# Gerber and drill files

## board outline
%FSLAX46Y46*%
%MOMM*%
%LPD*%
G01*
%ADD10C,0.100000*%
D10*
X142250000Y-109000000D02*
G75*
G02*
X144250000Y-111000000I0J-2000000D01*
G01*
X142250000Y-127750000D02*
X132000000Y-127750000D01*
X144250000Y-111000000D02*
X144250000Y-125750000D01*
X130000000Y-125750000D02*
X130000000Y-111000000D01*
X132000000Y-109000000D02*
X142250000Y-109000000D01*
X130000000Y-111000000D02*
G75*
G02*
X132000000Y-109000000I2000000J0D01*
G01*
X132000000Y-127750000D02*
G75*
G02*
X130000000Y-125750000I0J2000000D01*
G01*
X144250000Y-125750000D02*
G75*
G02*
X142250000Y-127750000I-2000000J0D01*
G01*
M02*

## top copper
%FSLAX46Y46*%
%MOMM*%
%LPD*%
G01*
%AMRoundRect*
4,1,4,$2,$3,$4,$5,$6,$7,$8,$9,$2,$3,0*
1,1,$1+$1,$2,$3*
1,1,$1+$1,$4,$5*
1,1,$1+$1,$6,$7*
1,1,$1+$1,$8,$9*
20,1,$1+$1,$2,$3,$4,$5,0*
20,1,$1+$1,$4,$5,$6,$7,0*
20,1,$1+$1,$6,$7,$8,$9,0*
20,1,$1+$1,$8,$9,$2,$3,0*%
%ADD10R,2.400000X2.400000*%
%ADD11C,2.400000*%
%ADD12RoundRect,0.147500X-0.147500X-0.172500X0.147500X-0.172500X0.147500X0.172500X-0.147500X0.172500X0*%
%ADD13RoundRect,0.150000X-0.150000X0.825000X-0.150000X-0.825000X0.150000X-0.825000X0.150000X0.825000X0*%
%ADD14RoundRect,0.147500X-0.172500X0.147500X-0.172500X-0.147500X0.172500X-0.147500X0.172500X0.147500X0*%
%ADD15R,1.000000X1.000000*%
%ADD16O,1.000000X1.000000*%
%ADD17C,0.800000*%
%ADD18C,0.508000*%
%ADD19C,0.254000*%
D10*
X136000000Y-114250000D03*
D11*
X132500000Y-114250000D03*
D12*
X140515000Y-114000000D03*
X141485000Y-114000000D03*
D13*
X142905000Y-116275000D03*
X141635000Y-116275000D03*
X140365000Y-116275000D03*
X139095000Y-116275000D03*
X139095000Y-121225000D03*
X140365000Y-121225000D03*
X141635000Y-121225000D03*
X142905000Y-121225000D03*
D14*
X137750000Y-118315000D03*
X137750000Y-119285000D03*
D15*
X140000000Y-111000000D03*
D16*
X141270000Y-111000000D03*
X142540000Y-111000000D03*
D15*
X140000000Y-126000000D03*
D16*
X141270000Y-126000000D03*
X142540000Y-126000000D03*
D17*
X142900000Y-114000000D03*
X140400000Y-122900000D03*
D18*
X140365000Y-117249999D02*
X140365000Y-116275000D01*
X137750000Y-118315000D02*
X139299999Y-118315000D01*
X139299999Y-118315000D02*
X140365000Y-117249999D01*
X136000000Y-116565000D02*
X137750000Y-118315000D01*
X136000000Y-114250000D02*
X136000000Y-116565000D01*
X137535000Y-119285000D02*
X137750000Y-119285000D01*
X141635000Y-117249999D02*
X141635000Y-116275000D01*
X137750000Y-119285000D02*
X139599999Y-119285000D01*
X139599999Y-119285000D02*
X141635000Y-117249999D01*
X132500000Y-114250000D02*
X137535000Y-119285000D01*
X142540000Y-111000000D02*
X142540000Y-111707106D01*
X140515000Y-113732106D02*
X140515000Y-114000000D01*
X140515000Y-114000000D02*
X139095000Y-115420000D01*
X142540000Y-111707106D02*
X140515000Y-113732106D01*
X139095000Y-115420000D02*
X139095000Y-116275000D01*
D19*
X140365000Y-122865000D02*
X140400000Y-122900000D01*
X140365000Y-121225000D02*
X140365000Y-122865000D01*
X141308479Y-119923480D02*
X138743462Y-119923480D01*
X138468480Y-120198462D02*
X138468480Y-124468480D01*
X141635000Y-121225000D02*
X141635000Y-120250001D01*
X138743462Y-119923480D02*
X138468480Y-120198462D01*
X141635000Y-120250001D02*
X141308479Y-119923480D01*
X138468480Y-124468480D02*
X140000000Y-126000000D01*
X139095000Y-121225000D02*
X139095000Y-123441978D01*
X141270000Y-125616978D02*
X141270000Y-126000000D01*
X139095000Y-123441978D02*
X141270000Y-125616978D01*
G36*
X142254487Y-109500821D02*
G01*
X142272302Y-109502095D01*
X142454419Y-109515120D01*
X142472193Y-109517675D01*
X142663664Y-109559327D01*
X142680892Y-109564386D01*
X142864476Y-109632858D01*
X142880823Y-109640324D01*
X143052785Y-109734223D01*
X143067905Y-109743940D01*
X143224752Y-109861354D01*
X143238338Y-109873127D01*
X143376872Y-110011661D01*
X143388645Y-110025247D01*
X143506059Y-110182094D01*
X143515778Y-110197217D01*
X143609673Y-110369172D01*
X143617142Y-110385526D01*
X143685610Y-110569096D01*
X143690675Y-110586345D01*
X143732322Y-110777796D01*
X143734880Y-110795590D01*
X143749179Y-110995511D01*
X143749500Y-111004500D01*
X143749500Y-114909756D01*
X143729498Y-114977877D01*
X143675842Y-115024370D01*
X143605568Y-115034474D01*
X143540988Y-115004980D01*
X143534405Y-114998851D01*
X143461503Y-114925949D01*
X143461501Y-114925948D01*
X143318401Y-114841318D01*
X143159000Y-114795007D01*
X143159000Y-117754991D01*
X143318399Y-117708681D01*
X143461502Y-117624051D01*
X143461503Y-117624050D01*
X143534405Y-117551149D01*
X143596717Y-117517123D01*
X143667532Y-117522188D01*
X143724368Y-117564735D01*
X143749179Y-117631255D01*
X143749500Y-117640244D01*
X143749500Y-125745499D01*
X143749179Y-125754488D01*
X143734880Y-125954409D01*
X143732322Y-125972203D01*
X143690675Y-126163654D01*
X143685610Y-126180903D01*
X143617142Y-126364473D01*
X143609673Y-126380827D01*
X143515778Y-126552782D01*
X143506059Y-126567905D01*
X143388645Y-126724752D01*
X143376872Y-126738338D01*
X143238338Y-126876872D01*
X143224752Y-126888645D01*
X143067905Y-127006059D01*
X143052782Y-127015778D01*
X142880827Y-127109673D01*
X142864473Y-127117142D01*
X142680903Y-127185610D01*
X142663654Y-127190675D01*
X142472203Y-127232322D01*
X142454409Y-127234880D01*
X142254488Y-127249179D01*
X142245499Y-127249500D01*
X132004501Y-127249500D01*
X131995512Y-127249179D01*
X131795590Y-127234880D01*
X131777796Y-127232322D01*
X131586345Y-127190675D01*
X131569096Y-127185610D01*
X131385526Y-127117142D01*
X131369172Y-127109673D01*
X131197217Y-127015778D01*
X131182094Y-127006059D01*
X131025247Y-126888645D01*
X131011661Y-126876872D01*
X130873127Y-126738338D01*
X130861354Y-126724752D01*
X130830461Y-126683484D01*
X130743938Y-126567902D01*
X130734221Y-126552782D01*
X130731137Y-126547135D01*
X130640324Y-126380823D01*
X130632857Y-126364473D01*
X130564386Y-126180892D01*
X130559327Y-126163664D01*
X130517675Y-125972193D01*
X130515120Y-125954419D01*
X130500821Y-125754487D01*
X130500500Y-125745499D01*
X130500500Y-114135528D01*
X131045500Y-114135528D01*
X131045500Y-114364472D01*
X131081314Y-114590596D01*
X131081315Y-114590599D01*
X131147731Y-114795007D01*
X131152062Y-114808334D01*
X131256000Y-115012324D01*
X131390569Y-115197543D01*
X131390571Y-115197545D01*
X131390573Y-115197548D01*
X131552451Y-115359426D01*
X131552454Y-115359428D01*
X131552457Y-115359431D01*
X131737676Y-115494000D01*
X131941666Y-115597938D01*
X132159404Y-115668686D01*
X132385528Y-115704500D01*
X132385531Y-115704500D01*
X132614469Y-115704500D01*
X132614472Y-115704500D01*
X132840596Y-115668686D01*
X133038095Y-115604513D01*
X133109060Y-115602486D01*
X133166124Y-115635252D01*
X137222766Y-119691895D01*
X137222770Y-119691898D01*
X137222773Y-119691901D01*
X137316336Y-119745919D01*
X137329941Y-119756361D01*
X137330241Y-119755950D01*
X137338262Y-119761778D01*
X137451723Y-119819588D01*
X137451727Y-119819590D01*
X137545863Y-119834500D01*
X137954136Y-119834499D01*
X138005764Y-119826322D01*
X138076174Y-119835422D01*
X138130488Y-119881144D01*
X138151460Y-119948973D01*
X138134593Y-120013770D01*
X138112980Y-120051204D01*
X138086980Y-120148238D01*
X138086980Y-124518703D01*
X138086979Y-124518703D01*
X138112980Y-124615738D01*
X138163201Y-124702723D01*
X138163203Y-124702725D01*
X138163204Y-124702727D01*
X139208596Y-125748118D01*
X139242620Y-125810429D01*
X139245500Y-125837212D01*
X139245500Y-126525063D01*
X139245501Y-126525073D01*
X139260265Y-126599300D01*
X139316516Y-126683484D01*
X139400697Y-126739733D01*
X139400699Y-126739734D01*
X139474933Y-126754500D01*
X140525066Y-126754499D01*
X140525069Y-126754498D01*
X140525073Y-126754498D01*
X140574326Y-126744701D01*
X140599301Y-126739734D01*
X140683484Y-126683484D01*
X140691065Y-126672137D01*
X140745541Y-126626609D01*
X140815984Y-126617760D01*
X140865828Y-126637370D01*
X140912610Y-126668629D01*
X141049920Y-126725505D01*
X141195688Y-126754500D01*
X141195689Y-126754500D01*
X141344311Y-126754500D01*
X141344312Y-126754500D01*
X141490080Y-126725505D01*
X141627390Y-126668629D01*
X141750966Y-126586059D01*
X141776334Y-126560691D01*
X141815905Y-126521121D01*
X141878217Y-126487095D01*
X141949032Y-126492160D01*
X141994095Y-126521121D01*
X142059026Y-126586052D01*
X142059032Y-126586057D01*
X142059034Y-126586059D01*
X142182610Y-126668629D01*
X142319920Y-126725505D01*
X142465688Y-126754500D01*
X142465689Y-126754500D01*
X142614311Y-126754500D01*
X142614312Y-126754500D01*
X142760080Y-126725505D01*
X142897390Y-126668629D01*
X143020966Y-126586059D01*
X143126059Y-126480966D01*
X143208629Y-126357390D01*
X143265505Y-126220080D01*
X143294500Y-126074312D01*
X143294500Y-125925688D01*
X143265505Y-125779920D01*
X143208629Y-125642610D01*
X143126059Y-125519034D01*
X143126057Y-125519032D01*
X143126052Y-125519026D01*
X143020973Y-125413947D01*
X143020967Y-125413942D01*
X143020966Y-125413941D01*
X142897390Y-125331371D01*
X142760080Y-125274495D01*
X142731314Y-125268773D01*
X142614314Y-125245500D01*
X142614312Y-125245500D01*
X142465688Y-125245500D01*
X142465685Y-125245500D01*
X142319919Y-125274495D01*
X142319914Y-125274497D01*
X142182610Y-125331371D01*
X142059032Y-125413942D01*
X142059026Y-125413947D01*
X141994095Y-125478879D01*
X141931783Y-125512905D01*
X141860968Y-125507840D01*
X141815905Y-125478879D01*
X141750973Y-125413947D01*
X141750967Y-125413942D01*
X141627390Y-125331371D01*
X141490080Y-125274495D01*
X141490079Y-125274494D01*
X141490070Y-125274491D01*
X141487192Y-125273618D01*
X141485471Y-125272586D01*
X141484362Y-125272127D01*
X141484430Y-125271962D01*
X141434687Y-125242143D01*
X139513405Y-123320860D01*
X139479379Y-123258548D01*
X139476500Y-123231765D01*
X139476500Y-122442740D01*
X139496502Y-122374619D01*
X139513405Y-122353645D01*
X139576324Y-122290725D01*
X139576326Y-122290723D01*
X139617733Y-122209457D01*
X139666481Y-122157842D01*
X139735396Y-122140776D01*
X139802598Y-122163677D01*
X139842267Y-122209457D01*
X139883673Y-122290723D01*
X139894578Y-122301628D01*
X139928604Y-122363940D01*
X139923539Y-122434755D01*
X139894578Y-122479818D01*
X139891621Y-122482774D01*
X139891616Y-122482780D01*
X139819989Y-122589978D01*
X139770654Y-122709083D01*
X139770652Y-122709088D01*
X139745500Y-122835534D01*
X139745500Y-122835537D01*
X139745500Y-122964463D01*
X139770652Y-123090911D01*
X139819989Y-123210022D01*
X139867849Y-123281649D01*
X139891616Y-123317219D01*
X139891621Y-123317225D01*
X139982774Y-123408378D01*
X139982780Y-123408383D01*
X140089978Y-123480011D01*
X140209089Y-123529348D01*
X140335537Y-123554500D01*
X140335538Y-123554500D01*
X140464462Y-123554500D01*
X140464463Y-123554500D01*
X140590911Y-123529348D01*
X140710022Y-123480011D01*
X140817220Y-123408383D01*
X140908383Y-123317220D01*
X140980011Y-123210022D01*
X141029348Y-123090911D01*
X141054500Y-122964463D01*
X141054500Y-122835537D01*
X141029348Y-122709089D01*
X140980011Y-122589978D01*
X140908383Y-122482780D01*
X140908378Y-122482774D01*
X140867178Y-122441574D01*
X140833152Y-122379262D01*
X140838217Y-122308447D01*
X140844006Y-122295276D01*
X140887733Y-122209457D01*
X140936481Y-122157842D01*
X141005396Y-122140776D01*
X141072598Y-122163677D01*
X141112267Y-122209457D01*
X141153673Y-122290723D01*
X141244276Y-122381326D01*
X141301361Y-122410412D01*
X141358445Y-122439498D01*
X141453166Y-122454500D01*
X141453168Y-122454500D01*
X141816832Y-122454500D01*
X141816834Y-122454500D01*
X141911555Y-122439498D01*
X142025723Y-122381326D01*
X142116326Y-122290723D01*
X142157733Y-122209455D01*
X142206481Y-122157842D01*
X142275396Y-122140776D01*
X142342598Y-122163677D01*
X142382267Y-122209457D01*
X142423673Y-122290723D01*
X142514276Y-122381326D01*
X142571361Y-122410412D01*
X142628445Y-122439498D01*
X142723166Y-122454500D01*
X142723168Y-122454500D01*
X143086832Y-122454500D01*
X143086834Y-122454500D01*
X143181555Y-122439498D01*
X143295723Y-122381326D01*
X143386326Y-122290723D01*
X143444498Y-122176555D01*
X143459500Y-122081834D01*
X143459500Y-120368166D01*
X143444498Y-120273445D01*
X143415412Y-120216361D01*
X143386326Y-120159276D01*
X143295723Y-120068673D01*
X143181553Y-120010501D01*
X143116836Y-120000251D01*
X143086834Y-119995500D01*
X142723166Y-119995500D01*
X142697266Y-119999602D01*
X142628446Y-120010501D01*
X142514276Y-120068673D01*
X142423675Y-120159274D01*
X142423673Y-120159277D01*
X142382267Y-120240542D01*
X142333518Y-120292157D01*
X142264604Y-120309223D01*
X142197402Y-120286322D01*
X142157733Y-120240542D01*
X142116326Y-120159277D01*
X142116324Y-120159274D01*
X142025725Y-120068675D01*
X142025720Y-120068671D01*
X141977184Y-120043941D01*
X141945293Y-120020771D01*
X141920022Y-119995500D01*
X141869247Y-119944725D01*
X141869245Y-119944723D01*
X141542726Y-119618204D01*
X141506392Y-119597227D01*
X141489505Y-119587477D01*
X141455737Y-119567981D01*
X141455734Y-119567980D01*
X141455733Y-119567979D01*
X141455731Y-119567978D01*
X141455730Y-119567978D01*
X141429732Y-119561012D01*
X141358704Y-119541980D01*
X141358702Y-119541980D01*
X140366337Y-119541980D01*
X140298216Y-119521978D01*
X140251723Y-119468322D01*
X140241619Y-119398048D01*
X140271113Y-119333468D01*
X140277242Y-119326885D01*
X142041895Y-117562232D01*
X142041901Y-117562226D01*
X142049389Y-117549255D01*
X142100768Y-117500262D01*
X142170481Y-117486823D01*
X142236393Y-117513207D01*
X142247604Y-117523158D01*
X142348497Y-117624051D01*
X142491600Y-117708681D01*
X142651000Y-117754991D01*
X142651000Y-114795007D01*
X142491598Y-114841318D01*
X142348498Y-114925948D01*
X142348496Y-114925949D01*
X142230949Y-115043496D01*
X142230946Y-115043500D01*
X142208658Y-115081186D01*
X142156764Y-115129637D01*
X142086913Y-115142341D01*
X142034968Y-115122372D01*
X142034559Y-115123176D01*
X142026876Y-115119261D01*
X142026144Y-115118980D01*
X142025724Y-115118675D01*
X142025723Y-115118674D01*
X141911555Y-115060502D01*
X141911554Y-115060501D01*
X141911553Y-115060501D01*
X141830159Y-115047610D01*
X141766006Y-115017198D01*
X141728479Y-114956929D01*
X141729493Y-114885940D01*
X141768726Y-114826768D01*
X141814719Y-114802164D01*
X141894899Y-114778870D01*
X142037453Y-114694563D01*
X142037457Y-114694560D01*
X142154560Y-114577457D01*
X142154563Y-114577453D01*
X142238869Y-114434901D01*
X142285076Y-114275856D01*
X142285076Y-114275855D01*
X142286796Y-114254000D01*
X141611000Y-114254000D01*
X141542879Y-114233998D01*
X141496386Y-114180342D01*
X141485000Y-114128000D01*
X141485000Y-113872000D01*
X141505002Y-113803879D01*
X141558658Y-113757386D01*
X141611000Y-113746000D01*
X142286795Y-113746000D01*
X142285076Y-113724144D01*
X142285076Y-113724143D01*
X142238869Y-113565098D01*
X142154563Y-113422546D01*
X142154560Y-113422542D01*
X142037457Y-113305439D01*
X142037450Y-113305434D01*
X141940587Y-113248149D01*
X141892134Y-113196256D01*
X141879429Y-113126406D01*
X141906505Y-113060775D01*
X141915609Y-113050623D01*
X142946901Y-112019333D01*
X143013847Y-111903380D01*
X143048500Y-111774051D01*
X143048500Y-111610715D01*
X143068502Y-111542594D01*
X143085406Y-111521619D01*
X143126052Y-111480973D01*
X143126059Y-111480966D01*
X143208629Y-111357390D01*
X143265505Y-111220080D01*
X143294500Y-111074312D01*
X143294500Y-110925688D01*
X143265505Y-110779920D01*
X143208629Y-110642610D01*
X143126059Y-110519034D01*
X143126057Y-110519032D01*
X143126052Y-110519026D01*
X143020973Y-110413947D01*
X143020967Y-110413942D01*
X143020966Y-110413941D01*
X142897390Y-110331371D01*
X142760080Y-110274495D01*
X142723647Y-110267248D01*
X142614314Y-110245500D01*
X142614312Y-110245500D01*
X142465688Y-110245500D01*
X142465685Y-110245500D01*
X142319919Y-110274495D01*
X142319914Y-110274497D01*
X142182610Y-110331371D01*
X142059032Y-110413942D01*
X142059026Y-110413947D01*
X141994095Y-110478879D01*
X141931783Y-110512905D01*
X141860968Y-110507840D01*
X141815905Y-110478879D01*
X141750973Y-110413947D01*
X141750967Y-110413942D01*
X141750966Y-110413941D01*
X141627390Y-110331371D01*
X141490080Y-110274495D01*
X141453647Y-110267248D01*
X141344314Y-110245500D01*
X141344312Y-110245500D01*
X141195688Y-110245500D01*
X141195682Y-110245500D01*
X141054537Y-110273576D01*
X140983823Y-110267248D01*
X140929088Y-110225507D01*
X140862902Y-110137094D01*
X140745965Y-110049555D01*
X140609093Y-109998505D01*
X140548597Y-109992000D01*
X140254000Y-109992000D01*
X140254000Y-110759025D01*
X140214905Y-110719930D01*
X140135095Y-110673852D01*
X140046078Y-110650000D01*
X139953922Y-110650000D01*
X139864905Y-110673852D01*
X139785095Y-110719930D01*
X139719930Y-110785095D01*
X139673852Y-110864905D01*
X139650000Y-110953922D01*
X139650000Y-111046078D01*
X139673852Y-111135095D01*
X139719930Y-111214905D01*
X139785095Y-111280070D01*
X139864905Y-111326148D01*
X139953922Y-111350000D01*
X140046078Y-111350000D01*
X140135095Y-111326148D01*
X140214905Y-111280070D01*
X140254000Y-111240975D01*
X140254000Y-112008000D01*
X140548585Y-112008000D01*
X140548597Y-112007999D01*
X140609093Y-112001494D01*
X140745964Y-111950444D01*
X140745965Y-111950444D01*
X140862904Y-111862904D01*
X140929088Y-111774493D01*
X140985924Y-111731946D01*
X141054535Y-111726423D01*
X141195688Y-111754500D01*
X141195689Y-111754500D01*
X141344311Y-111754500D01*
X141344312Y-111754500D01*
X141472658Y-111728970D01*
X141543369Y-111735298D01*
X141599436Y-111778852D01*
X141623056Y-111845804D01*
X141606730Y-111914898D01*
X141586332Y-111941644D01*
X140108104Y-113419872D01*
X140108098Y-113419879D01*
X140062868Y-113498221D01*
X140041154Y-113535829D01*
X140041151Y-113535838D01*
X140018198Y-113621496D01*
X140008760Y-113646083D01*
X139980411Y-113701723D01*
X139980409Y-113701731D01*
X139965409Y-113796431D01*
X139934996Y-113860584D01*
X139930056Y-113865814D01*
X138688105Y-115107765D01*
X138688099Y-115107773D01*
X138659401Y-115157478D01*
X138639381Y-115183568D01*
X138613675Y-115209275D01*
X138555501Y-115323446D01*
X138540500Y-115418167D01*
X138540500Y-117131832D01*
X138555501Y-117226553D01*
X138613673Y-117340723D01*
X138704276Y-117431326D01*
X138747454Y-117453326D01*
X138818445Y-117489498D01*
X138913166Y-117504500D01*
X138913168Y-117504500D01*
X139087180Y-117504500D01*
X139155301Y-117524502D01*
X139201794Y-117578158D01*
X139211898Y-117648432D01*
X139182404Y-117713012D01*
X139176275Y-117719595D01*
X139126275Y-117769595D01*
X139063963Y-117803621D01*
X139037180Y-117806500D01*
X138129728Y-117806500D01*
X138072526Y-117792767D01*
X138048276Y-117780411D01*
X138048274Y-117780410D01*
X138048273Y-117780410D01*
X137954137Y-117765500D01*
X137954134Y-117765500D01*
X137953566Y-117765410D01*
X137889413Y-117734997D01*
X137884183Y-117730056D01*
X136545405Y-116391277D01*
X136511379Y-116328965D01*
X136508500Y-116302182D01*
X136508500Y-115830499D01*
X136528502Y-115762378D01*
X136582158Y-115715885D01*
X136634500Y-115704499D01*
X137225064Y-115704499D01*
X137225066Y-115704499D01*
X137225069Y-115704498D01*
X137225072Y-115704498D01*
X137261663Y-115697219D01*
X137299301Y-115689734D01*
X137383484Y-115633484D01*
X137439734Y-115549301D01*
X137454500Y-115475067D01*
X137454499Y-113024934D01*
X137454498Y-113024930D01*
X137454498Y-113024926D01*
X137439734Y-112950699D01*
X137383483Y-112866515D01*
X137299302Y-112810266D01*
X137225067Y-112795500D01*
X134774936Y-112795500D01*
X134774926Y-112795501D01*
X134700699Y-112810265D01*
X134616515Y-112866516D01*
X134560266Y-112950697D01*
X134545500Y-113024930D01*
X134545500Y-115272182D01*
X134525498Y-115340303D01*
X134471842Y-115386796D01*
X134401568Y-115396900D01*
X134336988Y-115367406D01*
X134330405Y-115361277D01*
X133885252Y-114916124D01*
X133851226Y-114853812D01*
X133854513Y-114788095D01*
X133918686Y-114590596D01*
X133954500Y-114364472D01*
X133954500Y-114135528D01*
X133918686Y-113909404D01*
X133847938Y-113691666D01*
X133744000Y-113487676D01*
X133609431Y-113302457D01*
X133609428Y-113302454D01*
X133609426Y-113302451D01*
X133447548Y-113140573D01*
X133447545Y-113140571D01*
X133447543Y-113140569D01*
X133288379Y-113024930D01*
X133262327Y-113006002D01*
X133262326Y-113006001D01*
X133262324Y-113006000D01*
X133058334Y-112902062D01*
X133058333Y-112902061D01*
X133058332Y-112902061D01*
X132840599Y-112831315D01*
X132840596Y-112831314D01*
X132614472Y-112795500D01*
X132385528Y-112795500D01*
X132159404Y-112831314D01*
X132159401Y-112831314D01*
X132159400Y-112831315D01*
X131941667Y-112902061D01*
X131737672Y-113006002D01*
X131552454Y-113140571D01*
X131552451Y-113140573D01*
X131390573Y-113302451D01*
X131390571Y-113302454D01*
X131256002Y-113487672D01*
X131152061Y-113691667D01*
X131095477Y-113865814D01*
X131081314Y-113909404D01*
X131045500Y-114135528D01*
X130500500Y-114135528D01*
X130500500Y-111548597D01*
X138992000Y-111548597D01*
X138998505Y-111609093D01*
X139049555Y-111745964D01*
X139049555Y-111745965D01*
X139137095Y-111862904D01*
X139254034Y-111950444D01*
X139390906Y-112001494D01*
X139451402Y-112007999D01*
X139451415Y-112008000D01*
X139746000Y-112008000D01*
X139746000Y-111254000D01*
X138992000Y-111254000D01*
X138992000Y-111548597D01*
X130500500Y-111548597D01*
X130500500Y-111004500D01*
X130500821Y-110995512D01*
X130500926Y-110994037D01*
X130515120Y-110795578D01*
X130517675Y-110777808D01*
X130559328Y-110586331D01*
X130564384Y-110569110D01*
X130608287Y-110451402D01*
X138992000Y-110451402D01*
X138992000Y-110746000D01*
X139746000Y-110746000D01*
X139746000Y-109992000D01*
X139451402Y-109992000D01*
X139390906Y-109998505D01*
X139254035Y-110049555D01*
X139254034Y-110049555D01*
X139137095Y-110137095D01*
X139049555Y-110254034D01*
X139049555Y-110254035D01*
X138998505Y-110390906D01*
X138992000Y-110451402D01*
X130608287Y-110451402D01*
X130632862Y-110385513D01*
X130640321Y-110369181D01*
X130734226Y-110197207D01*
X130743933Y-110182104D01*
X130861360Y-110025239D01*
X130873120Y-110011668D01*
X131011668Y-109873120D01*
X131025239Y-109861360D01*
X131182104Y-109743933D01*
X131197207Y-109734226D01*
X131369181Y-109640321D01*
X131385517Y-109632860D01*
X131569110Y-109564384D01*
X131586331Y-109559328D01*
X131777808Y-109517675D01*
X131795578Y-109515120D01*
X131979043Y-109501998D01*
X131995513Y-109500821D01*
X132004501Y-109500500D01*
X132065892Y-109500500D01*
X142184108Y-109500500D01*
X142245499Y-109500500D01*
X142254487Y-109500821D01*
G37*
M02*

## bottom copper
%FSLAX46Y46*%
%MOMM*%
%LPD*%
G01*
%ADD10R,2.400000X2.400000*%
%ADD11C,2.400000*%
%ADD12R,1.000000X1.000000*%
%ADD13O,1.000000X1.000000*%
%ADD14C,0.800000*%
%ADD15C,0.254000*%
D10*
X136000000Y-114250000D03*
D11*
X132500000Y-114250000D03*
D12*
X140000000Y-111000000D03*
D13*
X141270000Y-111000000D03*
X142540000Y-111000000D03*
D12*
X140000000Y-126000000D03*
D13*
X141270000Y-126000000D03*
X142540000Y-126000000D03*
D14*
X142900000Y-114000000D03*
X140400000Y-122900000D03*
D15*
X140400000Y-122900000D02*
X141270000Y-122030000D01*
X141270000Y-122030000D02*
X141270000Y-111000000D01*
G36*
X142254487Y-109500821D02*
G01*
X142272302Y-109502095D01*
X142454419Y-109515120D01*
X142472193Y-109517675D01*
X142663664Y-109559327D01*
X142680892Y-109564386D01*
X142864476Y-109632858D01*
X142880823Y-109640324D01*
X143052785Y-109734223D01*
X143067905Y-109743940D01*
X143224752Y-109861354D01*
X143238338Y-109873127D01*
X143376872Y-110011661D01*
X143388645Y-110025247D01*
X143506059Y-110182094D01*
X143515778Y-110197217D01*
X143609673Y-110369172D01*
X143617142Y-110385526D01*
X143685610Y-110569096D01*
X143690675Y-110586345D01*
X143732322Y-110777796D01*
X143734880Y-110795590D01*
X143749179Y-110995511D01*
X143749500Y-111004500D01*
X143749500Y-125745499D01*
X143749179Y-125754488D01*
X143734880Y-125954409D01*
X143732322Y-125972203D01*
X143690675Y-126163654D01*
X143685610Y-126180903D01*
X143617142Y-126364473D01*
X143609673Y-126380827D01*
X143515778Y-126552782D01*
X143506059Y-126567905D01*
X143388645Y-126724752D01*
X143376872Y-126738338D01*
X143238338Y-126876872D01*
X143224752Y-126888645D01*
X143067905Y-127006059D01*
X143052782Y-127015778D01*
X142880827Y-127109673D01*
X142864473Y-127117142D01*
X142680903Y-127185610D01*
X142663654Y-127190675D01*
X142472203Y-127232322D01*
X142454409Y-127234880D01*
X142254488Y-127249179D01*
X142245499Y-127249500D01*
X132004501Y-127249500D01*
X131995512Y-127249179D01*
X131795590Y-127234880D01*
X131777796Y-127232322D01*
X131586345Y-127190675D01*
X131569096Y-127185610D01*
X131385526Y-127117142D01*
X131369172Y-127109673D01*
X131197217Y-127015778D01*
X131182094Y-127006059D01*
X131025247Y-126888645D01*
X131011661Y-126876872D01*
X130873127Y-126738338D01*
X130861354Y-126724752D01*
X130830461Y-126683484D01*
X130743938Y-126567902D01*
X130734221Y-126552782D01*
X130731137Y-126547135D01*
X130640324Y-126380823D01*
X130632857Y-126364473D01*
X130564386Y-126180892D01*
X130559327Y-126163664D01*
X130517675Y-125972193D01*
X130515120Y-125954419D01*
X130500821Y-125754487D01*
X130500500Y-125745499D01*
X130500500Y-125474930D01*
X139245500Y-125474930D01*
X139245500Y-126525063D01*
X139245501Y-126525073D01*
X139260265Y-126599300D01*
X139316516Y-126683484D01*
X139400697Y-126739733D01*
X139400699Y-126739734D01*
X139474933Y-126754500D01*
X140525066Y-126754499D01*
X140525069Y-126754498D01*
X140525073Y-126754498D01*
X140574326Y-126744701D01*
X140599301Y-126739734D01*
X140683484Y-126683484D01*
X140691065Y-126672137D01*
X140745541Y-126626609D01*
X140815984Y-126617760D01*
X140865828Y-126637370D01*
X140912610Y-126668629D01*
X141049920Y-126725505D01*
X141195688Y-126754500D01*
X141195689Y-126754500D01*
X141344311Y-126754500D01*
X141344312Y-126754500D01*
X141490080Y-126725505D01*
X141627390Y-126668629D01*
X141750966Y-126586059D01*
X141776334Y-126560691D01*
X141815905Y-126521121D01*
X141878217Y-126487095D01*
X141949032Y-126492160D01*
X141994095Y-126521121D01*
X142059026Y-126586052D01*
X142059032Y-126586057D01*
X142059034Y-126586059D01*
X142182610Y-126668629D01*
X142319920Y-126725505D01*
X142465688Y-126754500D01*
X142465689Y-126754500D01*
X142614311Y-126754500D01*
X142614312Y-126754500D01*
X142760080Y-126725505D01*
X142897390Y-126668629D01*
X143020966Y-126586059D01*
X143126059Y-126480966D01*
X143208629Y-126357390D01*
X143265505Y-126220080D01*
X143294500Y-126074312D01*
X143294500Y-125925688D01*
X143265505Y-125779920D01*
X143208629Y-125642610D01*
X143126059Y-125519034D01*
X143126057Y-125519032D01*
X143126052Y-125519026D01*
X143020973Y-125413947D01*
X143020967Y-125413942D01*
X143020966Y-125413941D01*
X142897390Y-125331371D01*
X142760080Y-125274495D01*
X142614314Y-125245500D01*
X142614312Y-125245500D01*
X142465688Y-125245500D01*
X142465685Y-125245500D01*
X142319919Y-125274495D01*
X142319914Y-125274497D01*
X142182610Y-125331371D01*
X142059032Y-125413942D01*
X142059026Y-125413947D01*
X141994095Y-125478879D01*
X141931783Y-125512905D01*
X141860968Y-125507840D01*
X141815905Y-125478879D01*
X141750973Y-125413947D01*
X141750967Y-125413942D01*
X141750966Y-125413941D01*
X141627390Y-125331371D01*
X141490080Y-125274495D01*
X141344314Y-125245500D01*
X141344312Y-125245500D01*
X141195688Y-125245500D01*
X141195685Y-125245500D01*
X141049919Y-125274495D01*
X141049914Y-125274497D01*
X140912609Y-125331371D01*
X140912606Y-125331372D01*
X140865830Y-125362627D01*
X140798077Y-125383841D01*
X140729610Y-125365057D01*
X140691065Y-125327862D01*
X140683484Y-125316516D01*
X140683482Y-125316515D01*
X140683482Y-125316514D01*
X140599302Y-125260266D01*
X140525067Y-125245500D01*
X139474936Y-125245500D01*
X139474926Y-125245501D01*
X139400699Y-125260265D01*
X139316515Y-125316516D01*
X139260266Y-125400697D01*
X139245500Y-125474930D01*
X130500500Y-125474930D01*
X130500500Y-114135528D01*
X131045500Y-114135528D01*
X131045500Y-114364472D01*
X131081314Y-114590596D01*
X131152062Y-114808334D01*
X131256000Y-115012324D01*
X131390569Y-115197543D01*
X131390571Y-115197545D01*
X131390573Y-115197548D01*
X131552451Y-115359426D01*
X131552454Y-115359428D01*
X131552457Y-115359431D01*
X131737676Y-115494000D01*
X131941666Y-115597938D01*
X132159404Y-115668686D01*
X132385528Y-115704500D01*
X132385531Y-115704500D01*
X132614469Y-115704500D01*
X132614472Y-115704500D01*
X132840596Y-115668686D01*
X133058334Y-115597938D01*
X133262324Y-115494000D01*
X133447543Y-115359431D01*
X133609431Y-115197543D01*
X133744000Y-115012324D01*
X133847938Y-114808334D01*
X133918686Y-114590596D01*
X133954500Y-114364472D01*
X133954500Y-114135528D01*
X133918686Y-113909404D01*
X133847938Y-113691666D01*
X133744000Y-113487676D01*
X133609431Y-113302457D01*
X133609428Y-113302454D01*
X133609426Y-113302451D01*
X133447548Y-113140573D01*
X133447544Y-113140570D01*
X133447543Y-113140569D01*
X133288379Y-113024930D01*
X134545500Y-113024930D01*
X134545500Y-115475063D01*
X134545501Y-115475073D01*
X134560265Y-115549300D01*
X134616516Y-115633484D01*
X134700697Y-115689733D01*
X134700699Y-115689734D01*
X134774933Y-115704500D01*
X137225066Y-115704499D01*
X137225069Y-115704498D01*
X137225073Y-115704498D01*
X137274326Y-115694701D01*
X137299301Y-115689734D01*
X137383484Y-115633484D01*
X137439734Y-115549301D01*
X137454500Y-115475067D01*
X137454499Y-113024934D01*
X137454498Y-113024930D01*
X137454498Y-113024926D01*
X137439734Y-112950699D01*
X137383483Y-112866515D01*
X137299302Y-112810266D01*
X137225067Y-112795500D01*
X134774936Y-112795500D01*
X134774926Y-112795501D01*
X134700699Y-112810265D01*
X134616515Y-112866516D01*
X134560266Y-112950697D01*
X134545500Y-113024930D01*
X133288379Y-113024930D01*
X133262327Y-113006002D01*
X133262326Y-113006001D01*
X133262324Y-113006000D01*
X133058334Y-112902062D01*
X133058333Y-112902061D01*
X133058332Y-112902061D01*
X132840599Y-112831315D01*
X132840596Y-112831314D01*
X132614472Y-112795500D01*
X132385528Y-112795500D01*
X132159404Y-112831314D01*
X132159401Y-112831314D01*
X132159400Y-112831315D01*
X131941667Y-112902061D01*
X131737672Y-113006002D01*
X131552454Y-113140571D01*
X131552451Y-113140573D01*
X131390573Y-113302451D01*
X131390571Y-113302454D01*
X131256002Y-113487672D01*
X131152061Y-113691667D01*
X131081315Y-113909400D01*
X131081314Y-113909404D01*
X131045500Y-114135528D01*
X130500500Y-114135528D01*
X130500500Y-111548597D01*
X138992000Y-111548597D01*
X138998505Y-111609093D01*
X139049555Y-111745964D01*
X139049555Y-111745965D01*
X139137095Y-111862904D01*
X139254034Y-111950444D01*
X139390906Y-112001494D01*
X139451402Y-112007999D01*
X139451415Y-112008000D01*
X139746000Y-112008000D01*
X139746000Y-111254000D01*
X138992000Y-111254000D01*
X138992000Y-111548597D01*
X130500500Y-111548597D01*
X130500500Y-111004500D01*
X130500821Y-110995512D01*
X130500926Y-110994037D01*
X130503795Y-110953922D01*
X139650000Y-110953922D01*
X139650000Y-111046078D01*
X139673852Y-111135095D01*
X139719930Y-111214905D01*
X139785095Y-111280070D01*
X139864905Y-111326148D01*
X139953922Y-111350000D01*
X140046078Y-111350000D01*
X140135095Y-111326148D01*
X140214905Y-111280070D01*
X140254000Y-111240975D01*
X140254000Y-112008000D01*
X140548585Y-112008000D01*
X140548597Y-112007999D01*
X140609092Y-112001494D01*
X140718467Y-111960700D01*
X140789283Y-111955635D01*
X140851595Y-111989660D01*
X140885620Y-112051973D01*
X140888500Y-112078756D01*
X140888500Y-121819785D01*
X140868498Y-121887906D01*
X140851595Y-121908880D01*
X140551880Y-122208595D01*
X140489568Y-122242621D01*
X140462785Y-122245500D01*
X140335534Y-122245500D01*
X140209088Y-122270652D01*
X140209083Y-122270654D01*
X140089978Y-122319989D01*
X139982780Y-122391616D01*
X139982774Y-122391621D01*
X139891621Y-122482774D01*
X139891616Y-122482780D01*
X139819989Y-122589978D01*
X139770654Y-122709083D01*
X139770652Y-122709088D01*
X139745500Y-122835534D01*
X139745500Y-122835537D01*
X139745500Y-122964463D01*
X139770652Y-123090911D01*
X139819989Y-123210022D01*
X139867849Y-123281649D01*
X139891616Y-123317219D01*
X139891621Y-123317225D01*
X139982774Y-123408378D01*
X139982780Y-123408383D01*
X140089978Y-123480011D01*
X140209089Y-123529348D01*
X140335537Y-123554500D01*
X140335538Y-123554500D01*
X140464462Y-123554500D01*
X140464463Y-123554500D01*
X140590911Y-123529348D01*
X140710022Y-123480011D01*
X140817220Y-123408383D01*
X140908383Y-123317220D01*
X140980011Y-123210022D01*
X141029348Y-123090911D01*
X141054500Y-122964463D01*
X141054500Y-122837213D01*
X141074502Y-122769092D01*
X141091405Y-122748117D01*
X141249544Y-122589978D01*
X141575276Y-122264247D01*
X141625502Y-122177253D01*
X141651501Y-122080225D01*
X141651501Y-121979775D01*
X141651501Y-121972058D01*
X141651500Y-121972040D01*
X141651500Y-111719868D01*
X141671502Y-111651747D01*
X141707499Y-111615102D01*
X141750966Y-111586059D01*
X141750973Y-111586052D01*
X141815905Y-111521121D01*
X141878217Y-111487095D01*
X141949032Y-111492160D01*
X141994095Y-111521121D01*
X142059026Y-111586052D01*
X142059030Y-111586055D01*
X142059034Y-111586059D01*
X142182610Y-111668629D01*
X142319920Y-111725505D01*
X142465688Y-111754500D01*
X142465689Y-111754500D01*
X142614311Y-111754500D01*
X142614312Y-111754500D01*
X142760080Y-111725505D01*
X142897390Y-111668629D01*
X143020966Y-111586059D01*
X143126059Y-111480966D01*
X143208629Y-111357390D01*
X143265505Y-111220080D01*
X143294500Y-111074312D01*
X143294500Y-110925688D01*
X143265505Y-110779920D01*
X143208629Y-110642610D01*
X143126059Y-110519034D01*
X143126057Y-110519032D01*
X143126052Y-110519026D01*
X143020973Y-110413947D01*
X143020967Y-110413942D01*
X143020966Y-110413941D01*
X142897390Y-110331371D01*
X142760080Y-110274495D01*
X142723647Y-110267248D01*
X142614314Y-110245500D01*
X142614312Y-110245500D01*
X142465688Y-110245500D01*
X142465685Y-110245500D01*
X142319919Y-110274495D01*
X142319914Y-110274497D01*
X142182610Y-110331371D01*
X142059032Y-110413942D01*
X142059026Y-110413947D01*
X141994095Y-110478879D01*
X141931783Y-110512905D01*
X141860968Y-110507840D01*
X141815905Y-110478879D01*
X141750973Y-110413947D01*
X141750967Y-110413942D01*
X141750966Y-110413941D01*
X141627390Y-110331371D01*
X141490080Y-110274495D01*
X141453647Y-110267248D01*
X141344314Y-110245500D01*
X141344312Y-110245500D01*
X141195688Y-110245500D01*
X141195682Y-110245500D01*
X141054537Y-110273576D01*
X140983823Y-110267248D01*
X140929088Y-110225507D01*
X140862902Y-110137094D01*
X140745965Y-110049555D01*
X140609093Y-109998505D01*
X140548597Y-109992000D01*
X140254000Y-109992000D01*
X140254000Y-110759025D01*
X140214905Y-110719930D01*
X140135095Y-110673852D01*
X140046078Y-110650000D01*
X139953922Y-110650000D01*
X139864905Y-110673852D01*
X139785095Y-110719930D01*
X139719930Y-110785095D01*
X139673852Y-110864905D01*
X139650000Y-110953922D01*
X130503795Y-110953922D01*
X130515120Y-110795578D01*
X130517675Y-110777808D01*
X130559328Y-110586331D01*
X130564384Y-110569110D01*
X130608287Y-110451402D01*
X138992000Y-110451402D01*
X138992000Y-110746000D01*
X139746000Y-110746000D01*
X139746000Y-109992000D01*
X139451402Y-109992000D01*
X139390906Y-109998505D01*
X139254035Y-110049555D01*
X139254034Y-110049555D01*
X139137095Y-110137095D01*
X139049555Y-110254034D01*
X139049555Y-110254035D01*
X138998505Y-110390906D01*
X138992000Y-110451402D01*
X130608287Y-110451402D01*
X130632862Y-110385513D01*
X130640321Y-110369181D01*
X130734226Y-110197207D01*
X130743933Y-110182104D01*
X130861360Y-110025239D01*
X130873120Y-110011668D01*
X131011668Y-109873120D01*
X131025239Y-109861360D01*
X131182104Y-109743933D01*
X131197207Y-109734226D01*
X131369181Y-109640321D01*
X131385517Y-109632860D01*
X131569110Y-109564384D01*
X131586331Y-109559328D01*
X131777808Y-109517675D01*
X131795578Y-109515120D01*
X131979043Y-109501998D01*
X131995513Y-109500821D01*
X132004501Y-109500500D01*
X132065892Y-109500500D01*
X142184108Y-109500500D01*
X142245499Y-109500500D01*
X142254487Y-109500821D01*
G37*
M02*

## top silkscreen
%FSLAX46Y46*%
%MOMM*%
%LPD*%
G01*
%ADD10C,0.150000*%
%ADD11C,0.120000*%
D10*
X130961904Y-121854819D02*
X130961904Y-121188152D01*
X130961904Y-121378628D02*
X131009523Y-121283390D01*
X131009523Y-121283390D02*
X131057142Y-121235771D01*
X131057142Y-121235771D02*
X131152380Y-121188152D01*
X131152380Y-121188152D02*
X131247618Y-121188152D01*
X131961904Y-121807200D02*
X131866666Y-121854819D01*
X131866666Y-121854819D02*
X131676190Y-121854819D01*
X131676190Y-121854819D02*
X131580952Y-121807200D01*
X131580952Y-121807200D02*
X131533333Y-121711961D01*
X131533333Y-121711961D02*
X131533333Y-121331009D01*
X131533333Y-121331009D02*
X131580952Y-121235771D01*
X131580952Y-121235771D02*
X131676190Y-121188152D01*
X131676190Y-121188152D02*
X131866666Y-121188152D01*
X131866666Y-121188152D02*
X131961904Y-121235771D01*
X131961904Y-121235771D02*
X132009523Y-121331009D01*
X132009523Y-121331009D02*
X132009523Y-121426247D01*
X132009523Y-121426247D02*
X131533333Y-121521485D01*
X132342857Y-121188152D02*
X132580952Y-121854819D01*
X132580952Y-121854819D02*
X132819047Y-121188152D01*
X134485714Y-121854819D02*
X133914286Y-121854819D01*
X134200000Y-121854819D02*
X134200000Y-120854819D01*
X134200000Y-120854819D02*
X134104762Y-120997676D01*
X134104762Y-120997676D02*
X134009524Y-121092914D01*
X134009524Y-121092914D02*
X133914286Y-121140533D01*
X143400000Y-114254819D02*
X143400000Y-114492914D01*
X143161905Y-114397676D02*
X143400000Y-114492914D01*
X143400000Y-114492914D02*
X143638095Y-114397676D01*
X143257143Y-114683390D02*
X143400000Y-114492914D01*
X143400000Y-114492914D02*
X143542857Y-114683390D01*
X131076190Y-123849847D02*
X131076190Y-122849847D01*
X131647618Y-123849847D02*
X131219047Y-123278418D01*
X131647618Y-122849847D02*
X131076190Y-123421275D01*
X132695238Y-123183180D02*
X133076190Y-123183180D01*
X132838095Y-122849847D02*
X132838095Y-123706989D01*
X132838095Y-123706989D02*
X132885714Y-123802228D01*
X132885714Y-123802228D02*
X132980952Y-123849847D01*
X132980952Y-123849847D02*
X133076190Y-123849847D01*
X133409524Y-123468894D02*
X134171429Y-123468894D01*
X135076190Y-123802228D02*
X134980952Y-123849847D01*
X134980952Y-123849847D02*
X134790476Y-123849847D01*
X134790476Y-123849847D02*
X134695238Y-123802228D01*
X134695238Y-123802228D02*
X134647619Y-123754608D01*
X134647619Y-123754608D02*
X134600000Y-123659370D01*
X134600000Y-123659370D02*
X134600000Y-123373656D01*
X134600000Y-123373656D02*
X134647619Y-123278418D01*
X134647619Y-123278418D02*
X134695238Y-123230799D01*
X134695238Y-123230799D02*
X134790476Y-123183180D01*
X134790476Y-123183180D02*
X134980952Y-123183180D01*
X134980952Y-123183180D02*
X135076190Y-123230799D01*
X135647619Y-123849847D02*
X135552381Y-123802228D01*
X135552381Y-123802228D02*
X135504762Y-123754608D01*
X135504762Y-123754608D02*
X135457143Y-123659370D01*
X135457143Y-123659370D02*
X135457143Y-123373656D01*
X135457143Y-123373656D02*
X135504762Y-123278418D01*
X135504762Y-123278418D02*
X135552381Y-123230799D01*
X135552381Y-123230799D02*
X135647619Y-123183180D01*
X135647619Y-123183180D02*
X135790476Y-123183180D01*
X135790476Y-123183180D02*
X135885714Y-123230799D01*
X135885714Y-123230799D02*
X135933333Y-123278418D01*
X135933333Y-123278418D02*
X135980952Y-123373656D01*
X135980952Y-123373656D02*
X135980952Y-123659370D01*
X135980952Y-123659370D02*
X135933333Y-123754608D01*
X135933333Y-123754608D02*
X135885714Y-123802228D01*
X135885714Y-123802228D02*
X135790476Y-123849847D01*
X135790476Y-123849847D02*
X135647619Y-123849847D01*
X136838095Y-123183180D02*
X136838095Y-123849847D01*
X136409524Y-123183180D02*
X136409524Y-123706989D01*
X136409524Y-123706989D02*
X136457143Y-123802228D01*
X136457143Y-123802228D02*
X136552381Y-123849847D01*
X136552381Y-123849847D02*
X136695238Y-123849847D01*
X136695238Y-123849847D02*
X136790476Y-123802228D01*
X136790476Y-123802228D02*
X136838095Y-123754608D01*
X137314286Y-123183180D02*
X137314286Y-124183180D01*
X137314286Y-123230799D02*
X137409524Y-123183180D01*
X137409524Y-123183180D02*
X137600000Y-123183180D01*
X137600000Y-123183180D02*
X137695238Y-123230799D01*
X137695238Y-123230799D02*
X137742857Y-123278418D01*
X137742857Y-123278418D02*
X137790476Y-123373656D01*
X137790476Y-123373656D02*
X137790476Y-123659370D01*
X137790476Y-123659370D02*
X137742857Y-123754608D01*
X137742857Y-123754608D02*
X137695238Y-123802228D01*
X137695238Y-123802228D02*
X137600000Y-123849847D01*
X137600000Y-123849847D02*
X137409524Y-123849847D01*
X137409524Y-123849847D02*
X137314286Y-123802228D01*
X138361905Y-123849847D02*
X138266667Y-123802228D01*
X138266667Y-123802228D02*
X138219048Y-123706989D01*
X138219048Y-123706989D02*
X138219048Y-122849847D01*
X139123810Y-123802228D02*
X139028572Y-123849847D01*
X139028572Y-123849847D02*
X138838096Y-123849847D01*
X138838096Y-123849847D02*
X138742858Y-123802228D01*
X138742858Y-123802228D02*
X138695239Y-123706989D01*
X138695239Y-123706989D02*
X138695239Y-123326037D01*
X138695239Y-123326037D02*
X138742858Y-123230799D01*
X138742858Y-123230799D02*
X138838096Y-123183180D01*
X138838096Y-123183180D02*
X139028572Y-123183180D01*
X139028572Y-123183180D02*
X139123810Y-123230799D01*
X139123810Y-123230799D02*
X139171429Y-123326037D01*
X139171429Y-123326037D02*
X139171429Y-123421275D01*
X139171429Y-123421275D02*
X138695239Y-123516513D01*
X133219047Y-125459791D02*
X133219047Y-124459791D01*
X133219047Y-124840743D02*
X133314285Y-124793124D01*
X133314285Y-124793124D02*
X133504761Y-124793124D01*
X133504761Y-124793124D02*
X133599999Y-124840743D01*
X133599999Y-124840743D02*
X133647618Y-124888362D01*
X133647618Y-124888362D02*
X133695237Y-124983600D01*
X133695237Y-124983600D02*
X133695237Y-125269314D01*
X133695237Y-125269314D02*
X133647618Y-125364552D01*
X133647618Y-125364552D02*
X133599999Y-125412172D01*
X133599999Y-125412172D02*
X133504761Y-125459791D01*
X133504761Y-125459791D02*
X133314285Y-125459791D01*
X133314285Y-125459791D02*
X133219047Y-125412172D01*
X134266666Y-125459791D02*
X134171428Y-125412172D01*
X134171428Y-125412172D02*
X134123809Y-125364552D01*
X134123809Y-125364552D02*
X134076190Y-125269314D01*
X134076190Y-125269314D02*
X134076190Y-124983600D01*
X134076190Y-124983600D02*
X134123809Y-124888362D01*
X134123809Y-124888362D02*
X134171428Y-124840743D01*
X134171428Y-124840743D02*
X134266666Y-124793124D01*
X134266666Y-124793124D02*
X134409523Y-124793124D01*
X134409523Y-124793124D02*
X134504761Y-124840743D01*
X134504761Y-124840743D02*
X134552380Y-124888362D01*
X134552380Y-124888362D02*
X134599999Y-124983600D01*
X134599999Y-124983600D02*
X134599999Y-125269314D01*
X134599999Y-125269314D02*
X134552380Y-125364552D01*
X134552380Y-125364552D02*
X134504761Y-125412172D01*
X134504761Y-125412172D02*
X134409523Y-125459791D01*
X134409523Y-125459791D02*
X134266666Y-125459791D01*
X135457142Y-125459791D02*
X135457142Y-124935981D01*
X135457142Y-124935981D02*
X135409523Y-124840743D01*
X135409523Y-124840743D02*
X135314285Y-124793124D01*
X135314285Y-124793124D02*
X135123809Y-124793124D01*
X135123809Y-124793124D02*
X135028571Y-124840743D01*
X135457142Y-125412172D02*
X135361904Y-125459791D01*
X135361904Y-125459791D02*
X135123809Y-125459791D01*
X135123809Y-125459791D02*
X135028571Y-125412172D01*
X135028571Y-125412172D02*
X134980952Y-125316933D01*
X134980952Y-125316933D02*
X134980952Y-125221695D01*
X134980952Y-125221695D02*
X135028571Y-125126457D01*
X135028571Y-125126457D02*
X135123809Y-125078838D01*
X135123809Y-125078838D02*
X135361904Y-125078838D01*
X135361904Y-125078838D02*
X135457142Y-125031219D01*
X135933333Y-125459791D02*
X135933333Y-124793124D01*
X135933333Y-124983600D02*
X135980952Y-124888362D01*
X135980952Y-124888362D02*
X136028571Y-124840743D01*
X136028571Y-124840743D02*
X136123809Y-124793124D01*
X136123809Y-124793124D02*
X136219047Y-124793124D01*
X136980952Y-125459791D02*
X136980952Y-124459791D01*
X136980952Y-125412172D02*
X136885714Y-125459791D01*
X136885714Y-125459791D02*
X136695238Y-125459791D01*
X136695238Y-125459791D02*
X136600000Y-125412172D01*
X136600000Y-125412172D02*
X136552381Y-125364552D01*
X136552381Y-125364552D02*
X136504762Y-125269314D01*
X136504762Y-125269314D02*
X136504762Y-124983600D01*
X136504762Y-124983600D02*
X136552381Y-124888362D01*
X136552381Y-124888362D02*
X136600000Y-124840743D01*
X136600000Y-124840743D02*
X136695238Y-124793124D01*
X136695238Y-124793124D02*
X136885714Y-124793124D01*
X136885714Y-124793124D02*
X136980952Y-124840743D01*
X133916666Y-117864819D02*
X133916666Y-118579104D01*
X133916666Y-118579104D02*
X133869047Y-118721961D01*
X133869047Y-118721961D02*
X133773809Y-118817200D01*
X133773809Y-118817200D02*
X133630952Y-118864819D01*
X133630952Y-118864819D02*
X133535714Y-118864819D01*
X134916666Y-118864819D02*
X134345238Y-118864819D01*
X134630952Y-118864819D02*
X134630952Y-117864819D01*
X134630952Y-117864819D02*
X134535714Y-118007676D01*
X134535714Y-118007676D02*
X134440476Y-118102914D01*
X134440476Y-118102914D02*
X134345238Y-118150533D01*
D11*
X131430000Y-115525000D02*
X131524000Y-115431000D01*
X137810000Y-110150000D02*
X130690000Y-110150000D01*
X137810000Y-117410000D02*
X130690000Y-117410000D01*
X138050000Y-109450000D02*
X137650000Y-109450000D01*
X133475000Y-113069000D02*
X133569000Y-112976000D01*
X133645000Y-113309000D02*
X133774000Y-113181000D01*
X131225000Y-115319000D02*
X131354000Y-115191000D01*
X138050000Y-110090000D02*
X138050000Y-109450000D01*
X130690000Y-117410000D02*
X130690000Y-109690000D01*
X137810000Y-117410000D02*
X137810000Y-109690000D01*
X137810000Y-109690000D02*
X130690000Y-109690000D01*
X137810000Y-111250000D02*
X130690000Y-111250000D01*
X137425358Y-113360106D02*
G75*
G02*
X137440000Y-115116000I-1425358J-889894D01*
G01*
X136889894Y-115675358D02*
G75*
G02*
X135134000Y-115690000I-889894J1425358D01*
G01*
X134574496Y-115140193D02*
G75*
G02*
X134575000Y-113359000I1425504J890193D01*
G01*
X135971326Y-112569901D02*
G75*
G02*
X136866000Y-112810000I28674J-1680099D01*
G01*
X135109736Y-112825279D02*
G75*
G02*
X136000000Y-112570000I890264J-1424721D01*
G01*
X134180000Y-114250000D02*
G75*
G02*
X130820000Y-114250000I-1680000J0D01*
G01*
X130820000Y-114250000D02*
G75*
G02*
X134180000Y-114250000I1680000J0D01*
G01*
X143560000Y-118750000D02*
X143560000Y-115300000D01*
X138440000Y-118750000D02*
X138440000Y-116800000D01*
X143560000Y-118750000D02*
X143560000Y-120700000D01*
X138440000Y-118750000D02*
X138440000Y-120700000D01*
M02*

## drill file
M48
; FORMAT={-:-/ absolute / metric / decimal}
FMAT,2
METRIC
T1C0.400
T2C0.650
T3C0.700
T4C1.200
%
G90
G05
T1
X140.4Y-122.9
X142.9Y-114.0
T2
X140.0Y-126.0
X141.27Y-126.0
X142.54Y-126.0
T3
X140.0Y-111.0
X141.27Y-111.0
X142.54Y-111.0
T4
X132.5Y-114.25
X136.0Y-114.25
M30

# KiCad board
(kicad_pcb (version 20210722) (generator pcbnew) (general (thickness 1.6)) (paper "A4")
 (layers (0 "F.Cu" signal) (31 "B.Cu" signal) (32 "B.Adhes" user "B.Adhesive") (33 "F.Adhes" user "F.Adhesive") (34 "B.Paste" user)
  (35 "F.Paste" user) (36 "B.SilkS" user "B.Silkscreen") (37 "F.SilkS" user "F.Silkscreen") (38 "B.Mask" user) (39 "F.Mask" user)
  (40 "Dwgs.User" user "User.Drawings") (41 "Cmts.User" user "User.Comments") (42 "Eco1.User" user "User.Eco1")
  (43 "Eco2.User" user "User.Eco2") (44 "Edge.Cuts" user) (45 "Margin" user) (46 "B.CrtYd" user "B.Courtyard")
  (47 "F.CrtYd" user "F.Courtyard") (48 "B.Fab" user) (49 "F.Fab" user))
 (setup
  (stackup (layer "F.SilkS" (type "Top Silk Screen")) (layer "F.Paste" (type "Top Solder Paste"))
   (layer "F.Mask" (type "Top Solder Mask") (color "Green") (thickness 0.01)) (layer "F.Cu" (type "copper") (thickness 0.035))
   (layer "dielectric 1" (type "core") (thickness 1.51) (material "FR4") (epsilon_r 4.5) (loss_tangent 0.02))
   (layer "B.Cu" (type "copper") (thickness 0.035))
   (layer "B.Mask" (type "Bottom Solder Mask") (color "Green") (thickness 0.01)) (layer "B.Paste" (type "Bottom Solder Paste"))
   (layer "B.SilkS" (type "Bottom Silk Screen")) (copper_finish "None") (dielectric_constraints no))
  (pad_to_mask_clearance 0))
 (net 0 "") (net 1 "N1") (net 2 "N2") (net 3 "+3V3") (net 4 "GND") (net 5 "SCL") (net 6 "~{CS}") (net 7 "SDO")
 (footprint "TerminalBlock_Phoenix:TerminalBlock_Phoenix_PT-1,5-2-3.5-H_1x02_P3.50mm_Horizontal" (layer "F.Cu") (at 136 114.25 180)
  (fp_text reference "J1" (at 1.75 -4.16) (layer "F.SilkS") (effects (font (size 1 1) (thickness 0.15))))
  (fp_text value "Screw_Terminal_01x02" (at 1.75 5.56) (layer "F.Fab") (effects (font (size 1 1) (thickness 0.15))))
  (fp_line (start 4.57 -1.275) (end 4.476 -1.181) (layer "F.SilkS") (width 0.12))
  (fp_line (start -1.81 4.1) (end 5.31 4.1) (layer "F.SilkS") (width 0.12))
  (fp_line (start -1.81 -3.16) (end 5.31 -3.16) (layer "F.SilkS") (width 0.12))
  (fp_line (start -2.05 4.8) (end -1.65 4.8) (layer "F.SilkS") (width 0.12))
  (fp_line (start 2.525 1.181) (end 2.431 1.274) (layer "F.SilkS") (width 0.12))
  (fp_line (start 2.355 0.941) (end 2.226 1.069) (layer "F.SilkS") (width 0.12))
  (fp_line (start 4.775 -1.069) (end 4.646 -0.941) (layer "F.SilkS") (width 0.12))
  (fp_line (start -2.05 4.16) (end -2.05 4.8) (layer "F.SilkS") (width 0.12))
  (fp_line (start 5.31 -3.16) (end 5.31 4.56) (layer "F.SilkS") (width 0.12))
  (fp_line (start -1.81 -3.16) (end -1.81 4.56) (layer "F.SilkS") (width 0.12))
  (fp_line (start -1.81 4.56) (end 5.31 4.56) (layer "F.SilkS") (width 0.12))
  (fp_line (start -1.81 3) (end 5.31 3) (layer "F.SilkS") (width 0.12))
  (fp_arc (start 0 0) (end -1.44 -0.866) (angle -63) (layer "F.SilkS") (width 0.12))
  (fp_arc (start 0 0) (end 0.866 -1.44) (angle -63) (layer "F.SilkS") (width 0.12))
  (fp_arc (start 0 0) (end 1.425 0.891) (angle -64) (layer "F.SilkS") (width 0.12))
  (fp_arc (start 0 0) (end -0.866 1.44) (angle -32) (layer "F.SilkS") (width 0.12))
  (fp_arc (start 0 0) (end 0 1.68) (angle -32) (layer "F.SilkS") (width 0.12))
  (fp_circle (center 3.5 0) (end 5.18 0) (layer "F.SilkS") (width 0.12) (fill none))
  (pad "1" thru_hole rect locked (at 0 0 180) (size 2.4 2.4) (drill 1.2) (layers *.Cu *.Mask) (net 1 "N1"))
  (pad "2" thru_hole circle locked (at 3.5 0 180) (size 2.4 2.4) (drill 1.2) (layers *.Cu *.Mask) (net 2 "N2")))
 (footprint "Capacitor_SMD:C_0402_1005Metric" (layer "F.Cu") (at 141 114)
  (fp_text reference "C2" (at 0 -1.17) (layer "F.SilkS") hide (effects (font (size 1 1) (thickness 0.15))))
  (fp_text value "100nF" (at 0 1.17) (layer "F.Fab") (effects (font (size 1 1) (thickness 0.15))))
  (pad "1" smd roundrect locked (at -0.485 0) (size 0.59 0.64) (layers "F.Cu" "F.Paste" "F.Mask") (roundrect_rratio 0.25) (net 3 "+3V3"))
  (pad "2" smd roundrect locked (at 0.485 0) (size 0.59 0.64) (layers "F.Cu" "F.Paste" "F.Mask") (roundrect_rratio 0.25) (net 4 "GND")))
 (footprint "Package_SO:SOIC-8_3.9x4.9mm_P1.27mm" (layer "F.Cu") (at 141 118.75 -90)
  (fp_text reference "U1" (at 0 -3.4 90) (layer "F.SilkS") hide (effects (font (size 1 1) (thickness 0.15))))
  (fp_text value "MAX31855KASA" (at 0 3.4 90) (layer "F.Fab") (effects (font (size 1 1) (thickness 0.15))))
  (fp_line (start 0 -2.56) (end -3.45 -2.56) (layer "F.SilkS") (width 0.12))
  (fp_line (start 0 2.56) (end -1.95 2.56) (layer "F.SilkS") (width 0.12))
  (fp_line (start 0 -2.56) (end 1.95 -2.56) (layer "F.SilkS") (width 0.12))
  (fp_line (start 0 2.56) (end 1.95 2.56) (layer "F.SilkS") (width 0.12))
  (pad "1" smd roundrect locked (at -2.475 -1.905 270) (size 1.95 0.6) (layers "F.Cu" "F.Paste" "F.Mask") (roundrect_rratio 0.25)
   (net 4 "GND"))
  (pad "2" smd roundrect locked (at -2.475 -0.635 270) (size 1.95 0.6) (layers "F.Cu" "F.Paste" "F.Mask") (roundrect_rratio 0.25)
   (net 2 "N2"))
  (pad "3" smd roundrect locked (at -2.475 0.635 270) (size 1.95 0.6) (layers "F.Cu" "F.Paste" "F.Mask") (roundrect_rratio 0.25)
   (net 1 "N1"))
  (pad "4" smd roundrect locked (at -2.475 1.905 270) (size 1.95 0.6) (layers "F.Cu" "F.Paste" "F.Mask") (roundrect_rratio 0.25)
   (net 3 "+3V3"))
  (pad "5" smd roundrect locked (at 2.475 1.905 270) (size 1.95 0.6) (layers "F.Cu" "F.Paste" "F.Mask") (roundrect_rratio 0.25)
   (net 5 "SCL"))
  (pad "6" smd roundrect locked (at 2.475 0.635 270) (size 1.95 0.6) (layers "F.Cu" "F.Paste" "F.Mask") (roundrect_rratio 0.25)
   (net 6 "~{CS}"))
  (pad "7" smd roundrect locked (at 2.475 -0.635 270) (size 1.95 0.6) (layers "F.Cu" "F.Paste" "F.Mask") (roundrect_rratio 0.25)
   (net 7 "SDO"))
  (pad "8" smd roundrect locked (at 2.475 -1.905 270) (size 1.95 0.6) (layers "F.Cu" "F.Paste" "F.Mask") (roundrect_rratio 0.25)))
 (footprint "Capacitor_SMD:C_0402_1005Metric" (layer "F.Cu") (at 137.75 118.8 -90)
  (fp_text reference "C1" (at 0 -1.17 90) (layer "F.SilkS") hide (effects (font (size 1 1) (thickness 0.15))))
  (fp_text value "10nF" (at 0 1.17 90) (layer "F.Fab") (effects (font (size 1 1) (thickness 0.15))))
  (pad "1" smd roundrect locked (at -0.485 0 270) (size 0.59 0.64) (layers "F.Cu" "F.Paste" "F.Mask") (roundrect_rratio 0.25) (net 1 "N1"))
  (pad "2" smd roundrect locked (at 0.485 0 270) (size 0.59 0.64) (layers "F.Cu" "F.Paste" "F.Mask") (roundrect_rratio 0.25) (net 2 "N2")))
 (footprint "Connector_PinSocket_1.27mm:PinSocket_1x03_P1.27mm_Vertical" (layer "B.Cu") (at 140 111 -90)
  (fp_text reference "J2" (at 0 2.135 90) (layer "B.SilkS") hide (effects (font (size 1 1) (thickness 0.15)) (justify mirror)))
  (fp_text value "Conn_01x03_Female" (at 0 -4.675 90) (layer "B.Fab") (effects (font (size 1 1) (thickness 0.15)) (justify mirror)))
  (pad "1" thru_hole rect locked (at 0 0 270) (size 1 1) (drill 0.7) (layers *.Cu *.Mask) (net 4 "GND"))
  (pad "2" thru_hole oval locked (at 0 -1.27 270) (size 1 1) (drill 0.7) (layers *.Cu *.Mask) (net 6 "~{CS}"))
  (pad "3" thru_hole oval locked (at 0 -2.54 270) (size 1 1) (drill 0.7) (layers *.Cu *.Mask) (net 3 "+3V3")))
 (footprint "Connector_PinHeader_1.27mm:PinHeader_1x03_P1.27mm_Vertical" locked (layer "B.Cu") (at 140 126 -90)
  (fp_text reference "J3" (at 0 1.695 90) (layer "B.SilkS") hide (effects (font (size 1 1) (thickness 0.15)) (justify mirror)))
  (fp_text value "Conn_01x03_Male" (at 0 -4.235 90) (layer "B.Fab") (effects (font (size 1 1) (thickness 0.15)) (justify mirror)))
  (pad "1" thru_hole rect locked (at 0 0 270) (size 1 1) (drill 0.65) (layers *.Cu *.Mask) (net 7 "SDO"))
  (pad "2" thru_hole oval locked (at 0 -1.27 270) (size 1 1) (drill 0.65) (layers *.Cu *.Mask) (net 5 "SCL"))
  (pad "3" thru_hole oval locked (at 0 -2.54 270) (size 1 1) (drill 0.65) (layers *.Cu *.Mask)))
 (gr_arc (start 142.25 111) (end 142.25 109) (angle 90) (layer "Edge.Cuts") (width 0.1))
 (gr_line (start 142.25 127.75) (end 132 127.75) (layer "Edge.Cuts") (width 0.1))
 (gr_line (start 144.25 111) (end 144.25 125.75) (layer "Edge.Cuts") (width 0.1))
 (gr_line (start 130 125.75) (end 130 111) (layer "Edge.Cuts") (width 0.1))
 (gr_line (start 132 109) (end 142.25 109) (layer "Edge.Cuts") (width 0.1))
 (gr_arc (start 132 111) (end 132 109) (angle -90) (layer "Edge.Cuts") (width 0.1))
 (gr_arc (start 132 125.75) (end 132 127.75) (angle 90) (layer "Edge.Cuts") (width 0.1))
 (gr_arc (start 142.25 125.75) (end 142.25 127.75) (angle -90) (layer "Edge.Cuts") (width 0.1))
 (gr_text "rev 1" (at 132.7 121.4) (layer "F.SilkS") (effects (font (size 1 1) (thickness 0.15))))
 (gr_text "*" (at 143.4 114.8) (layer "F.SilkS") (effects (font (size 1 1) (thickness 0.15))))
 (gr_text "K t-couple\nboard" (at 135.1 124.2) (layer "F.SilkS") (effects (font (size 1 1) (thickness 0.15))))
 (segment (start 140.365 117.249999) (end 140.365 116.275) (width 0.508) (layer "F.Cu") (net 1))
 (segment (start 137.75 118.315) (end 139.299999 118.315) (width 0.508) (layer "F.Cu") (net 1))
 (segment (start 139.299999 118.315) (end 140.365 117.249999) (width 0.508) (layer "F.Cu") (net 1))
 (segment (start 136 116.565) (end 137.75 118.315) (width 0.508) (layer "F.Cu") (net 1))
 (segment (start 136 114.25) (end 136 116.565) (width 0.508) (layer "F.Cu") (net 1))
 (segment (start 137.535 119.285) (end 137.75 119.285) (width 0.508) (layer "F.Cu") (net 2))
 (segment (start 141.635 117.249999) (end 141.635 116.275) (width 0.508) (layer "F.Cu") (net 2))
 (segment (start 137.75 119.285) (end 139.599999 119.285) (width 0.508) (layer "F.Cu") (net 2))
 (segment (start 139.599999 119.285) (end 141.635 117.249999) (width 0.508) (layer "F.Cu") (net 2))
 (segment (start 132.5 114.25) (end 137.535 119.285) (width 0.508) (layer "F.Cu") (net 2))
 (segment (start 142.54 111) (end 142.54 111.707106) (width 0.508) (layer "F.Cu") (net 3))
 (segment (start 140.515 113.732106) (end 140.515 114) (width 0.508) (layer "F.Cu") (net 3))
 (segment (start 140.515 114) (end 139.095 115.42) (width 0.508) (layer "F.Cu") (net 3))
 (segment (start 142.54 111.707106) (end 140.515 113.732106) (width 0.508) (layer "F.Cu") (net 3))
 (segment (start 139.095 115.42) (end 139.095 116.275) (width 0.508) (layer "F.Cu") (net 3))
 (via (at 142.9 114) (size 0.8) (drill 0.4) (layers "F.Cu" "B.Cu") (free) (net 4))
 (segment (start 140.365 122.865) (end 140.4 122.9) (width 0.254) (layer "F.Cu") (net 6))
 (segment (start 140.365 121.225) (end 140.365 122.865) (width 0.254) (layer "F.Cu") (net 6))
 (via (at 140.4 122.9) (size 0.8) (drill 0.4) (layers "F.Cu" "B.Cu") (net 6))
 (segment (start 140.4 122.9) (end 141.27 122.03) (width 0.254) (layer "B.Cu") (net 6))
 (segment (start 141.27 122.03) (end 141.27 111) (width 0.254) (layer "B.Cu") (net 6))
 (segment (start 141.308479 119.92348) (end 138.743462 119.92348) (width 0.254) (layer "F.Cu") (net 7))
 (segment (start 138.46848 120.198462) (end 138.46848 124.46848) (width 0.254) (layer "F.Cu") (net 7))
 (segment (start 141.635 121.225) (end 141.635 120.250001) (width 0.254) (layer "F.Cu") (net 7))
 (segment (start 138.743462 119.92348) (end 138.46848 120.198462) (width 0.254) (layer "F.Cu") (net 7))
 (segment (start 141.635 120.250001) (end 141.308479 119.92348) (width 0.254) (layer "F.Cu") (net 7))
 (segment (start 138.46848 124.46848) (end 140 126) (width 0.254) (layer "F.Cu") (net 7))
 (segment (start 139.095 121.225) (end 139.095 123.441978) (width 0.254) (layer "F.Cu") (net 5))
 (segment (start 141.27 125.616978) (end 141.27 126) (width 0.254) (layer "F.Cu") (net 5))
 (segment (start 139.095 123.441978) (end 141.27 125.616978) (width 0.254) (layer "F.Cu") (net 5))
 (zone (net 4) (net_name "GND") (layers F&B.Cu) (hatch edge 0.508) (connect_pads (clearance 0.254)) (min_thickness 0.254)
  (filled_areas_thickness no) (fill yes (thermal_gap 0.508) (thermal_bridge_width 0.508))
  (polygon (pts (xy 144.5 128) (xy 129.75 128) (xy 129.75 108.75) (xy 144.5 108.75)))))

